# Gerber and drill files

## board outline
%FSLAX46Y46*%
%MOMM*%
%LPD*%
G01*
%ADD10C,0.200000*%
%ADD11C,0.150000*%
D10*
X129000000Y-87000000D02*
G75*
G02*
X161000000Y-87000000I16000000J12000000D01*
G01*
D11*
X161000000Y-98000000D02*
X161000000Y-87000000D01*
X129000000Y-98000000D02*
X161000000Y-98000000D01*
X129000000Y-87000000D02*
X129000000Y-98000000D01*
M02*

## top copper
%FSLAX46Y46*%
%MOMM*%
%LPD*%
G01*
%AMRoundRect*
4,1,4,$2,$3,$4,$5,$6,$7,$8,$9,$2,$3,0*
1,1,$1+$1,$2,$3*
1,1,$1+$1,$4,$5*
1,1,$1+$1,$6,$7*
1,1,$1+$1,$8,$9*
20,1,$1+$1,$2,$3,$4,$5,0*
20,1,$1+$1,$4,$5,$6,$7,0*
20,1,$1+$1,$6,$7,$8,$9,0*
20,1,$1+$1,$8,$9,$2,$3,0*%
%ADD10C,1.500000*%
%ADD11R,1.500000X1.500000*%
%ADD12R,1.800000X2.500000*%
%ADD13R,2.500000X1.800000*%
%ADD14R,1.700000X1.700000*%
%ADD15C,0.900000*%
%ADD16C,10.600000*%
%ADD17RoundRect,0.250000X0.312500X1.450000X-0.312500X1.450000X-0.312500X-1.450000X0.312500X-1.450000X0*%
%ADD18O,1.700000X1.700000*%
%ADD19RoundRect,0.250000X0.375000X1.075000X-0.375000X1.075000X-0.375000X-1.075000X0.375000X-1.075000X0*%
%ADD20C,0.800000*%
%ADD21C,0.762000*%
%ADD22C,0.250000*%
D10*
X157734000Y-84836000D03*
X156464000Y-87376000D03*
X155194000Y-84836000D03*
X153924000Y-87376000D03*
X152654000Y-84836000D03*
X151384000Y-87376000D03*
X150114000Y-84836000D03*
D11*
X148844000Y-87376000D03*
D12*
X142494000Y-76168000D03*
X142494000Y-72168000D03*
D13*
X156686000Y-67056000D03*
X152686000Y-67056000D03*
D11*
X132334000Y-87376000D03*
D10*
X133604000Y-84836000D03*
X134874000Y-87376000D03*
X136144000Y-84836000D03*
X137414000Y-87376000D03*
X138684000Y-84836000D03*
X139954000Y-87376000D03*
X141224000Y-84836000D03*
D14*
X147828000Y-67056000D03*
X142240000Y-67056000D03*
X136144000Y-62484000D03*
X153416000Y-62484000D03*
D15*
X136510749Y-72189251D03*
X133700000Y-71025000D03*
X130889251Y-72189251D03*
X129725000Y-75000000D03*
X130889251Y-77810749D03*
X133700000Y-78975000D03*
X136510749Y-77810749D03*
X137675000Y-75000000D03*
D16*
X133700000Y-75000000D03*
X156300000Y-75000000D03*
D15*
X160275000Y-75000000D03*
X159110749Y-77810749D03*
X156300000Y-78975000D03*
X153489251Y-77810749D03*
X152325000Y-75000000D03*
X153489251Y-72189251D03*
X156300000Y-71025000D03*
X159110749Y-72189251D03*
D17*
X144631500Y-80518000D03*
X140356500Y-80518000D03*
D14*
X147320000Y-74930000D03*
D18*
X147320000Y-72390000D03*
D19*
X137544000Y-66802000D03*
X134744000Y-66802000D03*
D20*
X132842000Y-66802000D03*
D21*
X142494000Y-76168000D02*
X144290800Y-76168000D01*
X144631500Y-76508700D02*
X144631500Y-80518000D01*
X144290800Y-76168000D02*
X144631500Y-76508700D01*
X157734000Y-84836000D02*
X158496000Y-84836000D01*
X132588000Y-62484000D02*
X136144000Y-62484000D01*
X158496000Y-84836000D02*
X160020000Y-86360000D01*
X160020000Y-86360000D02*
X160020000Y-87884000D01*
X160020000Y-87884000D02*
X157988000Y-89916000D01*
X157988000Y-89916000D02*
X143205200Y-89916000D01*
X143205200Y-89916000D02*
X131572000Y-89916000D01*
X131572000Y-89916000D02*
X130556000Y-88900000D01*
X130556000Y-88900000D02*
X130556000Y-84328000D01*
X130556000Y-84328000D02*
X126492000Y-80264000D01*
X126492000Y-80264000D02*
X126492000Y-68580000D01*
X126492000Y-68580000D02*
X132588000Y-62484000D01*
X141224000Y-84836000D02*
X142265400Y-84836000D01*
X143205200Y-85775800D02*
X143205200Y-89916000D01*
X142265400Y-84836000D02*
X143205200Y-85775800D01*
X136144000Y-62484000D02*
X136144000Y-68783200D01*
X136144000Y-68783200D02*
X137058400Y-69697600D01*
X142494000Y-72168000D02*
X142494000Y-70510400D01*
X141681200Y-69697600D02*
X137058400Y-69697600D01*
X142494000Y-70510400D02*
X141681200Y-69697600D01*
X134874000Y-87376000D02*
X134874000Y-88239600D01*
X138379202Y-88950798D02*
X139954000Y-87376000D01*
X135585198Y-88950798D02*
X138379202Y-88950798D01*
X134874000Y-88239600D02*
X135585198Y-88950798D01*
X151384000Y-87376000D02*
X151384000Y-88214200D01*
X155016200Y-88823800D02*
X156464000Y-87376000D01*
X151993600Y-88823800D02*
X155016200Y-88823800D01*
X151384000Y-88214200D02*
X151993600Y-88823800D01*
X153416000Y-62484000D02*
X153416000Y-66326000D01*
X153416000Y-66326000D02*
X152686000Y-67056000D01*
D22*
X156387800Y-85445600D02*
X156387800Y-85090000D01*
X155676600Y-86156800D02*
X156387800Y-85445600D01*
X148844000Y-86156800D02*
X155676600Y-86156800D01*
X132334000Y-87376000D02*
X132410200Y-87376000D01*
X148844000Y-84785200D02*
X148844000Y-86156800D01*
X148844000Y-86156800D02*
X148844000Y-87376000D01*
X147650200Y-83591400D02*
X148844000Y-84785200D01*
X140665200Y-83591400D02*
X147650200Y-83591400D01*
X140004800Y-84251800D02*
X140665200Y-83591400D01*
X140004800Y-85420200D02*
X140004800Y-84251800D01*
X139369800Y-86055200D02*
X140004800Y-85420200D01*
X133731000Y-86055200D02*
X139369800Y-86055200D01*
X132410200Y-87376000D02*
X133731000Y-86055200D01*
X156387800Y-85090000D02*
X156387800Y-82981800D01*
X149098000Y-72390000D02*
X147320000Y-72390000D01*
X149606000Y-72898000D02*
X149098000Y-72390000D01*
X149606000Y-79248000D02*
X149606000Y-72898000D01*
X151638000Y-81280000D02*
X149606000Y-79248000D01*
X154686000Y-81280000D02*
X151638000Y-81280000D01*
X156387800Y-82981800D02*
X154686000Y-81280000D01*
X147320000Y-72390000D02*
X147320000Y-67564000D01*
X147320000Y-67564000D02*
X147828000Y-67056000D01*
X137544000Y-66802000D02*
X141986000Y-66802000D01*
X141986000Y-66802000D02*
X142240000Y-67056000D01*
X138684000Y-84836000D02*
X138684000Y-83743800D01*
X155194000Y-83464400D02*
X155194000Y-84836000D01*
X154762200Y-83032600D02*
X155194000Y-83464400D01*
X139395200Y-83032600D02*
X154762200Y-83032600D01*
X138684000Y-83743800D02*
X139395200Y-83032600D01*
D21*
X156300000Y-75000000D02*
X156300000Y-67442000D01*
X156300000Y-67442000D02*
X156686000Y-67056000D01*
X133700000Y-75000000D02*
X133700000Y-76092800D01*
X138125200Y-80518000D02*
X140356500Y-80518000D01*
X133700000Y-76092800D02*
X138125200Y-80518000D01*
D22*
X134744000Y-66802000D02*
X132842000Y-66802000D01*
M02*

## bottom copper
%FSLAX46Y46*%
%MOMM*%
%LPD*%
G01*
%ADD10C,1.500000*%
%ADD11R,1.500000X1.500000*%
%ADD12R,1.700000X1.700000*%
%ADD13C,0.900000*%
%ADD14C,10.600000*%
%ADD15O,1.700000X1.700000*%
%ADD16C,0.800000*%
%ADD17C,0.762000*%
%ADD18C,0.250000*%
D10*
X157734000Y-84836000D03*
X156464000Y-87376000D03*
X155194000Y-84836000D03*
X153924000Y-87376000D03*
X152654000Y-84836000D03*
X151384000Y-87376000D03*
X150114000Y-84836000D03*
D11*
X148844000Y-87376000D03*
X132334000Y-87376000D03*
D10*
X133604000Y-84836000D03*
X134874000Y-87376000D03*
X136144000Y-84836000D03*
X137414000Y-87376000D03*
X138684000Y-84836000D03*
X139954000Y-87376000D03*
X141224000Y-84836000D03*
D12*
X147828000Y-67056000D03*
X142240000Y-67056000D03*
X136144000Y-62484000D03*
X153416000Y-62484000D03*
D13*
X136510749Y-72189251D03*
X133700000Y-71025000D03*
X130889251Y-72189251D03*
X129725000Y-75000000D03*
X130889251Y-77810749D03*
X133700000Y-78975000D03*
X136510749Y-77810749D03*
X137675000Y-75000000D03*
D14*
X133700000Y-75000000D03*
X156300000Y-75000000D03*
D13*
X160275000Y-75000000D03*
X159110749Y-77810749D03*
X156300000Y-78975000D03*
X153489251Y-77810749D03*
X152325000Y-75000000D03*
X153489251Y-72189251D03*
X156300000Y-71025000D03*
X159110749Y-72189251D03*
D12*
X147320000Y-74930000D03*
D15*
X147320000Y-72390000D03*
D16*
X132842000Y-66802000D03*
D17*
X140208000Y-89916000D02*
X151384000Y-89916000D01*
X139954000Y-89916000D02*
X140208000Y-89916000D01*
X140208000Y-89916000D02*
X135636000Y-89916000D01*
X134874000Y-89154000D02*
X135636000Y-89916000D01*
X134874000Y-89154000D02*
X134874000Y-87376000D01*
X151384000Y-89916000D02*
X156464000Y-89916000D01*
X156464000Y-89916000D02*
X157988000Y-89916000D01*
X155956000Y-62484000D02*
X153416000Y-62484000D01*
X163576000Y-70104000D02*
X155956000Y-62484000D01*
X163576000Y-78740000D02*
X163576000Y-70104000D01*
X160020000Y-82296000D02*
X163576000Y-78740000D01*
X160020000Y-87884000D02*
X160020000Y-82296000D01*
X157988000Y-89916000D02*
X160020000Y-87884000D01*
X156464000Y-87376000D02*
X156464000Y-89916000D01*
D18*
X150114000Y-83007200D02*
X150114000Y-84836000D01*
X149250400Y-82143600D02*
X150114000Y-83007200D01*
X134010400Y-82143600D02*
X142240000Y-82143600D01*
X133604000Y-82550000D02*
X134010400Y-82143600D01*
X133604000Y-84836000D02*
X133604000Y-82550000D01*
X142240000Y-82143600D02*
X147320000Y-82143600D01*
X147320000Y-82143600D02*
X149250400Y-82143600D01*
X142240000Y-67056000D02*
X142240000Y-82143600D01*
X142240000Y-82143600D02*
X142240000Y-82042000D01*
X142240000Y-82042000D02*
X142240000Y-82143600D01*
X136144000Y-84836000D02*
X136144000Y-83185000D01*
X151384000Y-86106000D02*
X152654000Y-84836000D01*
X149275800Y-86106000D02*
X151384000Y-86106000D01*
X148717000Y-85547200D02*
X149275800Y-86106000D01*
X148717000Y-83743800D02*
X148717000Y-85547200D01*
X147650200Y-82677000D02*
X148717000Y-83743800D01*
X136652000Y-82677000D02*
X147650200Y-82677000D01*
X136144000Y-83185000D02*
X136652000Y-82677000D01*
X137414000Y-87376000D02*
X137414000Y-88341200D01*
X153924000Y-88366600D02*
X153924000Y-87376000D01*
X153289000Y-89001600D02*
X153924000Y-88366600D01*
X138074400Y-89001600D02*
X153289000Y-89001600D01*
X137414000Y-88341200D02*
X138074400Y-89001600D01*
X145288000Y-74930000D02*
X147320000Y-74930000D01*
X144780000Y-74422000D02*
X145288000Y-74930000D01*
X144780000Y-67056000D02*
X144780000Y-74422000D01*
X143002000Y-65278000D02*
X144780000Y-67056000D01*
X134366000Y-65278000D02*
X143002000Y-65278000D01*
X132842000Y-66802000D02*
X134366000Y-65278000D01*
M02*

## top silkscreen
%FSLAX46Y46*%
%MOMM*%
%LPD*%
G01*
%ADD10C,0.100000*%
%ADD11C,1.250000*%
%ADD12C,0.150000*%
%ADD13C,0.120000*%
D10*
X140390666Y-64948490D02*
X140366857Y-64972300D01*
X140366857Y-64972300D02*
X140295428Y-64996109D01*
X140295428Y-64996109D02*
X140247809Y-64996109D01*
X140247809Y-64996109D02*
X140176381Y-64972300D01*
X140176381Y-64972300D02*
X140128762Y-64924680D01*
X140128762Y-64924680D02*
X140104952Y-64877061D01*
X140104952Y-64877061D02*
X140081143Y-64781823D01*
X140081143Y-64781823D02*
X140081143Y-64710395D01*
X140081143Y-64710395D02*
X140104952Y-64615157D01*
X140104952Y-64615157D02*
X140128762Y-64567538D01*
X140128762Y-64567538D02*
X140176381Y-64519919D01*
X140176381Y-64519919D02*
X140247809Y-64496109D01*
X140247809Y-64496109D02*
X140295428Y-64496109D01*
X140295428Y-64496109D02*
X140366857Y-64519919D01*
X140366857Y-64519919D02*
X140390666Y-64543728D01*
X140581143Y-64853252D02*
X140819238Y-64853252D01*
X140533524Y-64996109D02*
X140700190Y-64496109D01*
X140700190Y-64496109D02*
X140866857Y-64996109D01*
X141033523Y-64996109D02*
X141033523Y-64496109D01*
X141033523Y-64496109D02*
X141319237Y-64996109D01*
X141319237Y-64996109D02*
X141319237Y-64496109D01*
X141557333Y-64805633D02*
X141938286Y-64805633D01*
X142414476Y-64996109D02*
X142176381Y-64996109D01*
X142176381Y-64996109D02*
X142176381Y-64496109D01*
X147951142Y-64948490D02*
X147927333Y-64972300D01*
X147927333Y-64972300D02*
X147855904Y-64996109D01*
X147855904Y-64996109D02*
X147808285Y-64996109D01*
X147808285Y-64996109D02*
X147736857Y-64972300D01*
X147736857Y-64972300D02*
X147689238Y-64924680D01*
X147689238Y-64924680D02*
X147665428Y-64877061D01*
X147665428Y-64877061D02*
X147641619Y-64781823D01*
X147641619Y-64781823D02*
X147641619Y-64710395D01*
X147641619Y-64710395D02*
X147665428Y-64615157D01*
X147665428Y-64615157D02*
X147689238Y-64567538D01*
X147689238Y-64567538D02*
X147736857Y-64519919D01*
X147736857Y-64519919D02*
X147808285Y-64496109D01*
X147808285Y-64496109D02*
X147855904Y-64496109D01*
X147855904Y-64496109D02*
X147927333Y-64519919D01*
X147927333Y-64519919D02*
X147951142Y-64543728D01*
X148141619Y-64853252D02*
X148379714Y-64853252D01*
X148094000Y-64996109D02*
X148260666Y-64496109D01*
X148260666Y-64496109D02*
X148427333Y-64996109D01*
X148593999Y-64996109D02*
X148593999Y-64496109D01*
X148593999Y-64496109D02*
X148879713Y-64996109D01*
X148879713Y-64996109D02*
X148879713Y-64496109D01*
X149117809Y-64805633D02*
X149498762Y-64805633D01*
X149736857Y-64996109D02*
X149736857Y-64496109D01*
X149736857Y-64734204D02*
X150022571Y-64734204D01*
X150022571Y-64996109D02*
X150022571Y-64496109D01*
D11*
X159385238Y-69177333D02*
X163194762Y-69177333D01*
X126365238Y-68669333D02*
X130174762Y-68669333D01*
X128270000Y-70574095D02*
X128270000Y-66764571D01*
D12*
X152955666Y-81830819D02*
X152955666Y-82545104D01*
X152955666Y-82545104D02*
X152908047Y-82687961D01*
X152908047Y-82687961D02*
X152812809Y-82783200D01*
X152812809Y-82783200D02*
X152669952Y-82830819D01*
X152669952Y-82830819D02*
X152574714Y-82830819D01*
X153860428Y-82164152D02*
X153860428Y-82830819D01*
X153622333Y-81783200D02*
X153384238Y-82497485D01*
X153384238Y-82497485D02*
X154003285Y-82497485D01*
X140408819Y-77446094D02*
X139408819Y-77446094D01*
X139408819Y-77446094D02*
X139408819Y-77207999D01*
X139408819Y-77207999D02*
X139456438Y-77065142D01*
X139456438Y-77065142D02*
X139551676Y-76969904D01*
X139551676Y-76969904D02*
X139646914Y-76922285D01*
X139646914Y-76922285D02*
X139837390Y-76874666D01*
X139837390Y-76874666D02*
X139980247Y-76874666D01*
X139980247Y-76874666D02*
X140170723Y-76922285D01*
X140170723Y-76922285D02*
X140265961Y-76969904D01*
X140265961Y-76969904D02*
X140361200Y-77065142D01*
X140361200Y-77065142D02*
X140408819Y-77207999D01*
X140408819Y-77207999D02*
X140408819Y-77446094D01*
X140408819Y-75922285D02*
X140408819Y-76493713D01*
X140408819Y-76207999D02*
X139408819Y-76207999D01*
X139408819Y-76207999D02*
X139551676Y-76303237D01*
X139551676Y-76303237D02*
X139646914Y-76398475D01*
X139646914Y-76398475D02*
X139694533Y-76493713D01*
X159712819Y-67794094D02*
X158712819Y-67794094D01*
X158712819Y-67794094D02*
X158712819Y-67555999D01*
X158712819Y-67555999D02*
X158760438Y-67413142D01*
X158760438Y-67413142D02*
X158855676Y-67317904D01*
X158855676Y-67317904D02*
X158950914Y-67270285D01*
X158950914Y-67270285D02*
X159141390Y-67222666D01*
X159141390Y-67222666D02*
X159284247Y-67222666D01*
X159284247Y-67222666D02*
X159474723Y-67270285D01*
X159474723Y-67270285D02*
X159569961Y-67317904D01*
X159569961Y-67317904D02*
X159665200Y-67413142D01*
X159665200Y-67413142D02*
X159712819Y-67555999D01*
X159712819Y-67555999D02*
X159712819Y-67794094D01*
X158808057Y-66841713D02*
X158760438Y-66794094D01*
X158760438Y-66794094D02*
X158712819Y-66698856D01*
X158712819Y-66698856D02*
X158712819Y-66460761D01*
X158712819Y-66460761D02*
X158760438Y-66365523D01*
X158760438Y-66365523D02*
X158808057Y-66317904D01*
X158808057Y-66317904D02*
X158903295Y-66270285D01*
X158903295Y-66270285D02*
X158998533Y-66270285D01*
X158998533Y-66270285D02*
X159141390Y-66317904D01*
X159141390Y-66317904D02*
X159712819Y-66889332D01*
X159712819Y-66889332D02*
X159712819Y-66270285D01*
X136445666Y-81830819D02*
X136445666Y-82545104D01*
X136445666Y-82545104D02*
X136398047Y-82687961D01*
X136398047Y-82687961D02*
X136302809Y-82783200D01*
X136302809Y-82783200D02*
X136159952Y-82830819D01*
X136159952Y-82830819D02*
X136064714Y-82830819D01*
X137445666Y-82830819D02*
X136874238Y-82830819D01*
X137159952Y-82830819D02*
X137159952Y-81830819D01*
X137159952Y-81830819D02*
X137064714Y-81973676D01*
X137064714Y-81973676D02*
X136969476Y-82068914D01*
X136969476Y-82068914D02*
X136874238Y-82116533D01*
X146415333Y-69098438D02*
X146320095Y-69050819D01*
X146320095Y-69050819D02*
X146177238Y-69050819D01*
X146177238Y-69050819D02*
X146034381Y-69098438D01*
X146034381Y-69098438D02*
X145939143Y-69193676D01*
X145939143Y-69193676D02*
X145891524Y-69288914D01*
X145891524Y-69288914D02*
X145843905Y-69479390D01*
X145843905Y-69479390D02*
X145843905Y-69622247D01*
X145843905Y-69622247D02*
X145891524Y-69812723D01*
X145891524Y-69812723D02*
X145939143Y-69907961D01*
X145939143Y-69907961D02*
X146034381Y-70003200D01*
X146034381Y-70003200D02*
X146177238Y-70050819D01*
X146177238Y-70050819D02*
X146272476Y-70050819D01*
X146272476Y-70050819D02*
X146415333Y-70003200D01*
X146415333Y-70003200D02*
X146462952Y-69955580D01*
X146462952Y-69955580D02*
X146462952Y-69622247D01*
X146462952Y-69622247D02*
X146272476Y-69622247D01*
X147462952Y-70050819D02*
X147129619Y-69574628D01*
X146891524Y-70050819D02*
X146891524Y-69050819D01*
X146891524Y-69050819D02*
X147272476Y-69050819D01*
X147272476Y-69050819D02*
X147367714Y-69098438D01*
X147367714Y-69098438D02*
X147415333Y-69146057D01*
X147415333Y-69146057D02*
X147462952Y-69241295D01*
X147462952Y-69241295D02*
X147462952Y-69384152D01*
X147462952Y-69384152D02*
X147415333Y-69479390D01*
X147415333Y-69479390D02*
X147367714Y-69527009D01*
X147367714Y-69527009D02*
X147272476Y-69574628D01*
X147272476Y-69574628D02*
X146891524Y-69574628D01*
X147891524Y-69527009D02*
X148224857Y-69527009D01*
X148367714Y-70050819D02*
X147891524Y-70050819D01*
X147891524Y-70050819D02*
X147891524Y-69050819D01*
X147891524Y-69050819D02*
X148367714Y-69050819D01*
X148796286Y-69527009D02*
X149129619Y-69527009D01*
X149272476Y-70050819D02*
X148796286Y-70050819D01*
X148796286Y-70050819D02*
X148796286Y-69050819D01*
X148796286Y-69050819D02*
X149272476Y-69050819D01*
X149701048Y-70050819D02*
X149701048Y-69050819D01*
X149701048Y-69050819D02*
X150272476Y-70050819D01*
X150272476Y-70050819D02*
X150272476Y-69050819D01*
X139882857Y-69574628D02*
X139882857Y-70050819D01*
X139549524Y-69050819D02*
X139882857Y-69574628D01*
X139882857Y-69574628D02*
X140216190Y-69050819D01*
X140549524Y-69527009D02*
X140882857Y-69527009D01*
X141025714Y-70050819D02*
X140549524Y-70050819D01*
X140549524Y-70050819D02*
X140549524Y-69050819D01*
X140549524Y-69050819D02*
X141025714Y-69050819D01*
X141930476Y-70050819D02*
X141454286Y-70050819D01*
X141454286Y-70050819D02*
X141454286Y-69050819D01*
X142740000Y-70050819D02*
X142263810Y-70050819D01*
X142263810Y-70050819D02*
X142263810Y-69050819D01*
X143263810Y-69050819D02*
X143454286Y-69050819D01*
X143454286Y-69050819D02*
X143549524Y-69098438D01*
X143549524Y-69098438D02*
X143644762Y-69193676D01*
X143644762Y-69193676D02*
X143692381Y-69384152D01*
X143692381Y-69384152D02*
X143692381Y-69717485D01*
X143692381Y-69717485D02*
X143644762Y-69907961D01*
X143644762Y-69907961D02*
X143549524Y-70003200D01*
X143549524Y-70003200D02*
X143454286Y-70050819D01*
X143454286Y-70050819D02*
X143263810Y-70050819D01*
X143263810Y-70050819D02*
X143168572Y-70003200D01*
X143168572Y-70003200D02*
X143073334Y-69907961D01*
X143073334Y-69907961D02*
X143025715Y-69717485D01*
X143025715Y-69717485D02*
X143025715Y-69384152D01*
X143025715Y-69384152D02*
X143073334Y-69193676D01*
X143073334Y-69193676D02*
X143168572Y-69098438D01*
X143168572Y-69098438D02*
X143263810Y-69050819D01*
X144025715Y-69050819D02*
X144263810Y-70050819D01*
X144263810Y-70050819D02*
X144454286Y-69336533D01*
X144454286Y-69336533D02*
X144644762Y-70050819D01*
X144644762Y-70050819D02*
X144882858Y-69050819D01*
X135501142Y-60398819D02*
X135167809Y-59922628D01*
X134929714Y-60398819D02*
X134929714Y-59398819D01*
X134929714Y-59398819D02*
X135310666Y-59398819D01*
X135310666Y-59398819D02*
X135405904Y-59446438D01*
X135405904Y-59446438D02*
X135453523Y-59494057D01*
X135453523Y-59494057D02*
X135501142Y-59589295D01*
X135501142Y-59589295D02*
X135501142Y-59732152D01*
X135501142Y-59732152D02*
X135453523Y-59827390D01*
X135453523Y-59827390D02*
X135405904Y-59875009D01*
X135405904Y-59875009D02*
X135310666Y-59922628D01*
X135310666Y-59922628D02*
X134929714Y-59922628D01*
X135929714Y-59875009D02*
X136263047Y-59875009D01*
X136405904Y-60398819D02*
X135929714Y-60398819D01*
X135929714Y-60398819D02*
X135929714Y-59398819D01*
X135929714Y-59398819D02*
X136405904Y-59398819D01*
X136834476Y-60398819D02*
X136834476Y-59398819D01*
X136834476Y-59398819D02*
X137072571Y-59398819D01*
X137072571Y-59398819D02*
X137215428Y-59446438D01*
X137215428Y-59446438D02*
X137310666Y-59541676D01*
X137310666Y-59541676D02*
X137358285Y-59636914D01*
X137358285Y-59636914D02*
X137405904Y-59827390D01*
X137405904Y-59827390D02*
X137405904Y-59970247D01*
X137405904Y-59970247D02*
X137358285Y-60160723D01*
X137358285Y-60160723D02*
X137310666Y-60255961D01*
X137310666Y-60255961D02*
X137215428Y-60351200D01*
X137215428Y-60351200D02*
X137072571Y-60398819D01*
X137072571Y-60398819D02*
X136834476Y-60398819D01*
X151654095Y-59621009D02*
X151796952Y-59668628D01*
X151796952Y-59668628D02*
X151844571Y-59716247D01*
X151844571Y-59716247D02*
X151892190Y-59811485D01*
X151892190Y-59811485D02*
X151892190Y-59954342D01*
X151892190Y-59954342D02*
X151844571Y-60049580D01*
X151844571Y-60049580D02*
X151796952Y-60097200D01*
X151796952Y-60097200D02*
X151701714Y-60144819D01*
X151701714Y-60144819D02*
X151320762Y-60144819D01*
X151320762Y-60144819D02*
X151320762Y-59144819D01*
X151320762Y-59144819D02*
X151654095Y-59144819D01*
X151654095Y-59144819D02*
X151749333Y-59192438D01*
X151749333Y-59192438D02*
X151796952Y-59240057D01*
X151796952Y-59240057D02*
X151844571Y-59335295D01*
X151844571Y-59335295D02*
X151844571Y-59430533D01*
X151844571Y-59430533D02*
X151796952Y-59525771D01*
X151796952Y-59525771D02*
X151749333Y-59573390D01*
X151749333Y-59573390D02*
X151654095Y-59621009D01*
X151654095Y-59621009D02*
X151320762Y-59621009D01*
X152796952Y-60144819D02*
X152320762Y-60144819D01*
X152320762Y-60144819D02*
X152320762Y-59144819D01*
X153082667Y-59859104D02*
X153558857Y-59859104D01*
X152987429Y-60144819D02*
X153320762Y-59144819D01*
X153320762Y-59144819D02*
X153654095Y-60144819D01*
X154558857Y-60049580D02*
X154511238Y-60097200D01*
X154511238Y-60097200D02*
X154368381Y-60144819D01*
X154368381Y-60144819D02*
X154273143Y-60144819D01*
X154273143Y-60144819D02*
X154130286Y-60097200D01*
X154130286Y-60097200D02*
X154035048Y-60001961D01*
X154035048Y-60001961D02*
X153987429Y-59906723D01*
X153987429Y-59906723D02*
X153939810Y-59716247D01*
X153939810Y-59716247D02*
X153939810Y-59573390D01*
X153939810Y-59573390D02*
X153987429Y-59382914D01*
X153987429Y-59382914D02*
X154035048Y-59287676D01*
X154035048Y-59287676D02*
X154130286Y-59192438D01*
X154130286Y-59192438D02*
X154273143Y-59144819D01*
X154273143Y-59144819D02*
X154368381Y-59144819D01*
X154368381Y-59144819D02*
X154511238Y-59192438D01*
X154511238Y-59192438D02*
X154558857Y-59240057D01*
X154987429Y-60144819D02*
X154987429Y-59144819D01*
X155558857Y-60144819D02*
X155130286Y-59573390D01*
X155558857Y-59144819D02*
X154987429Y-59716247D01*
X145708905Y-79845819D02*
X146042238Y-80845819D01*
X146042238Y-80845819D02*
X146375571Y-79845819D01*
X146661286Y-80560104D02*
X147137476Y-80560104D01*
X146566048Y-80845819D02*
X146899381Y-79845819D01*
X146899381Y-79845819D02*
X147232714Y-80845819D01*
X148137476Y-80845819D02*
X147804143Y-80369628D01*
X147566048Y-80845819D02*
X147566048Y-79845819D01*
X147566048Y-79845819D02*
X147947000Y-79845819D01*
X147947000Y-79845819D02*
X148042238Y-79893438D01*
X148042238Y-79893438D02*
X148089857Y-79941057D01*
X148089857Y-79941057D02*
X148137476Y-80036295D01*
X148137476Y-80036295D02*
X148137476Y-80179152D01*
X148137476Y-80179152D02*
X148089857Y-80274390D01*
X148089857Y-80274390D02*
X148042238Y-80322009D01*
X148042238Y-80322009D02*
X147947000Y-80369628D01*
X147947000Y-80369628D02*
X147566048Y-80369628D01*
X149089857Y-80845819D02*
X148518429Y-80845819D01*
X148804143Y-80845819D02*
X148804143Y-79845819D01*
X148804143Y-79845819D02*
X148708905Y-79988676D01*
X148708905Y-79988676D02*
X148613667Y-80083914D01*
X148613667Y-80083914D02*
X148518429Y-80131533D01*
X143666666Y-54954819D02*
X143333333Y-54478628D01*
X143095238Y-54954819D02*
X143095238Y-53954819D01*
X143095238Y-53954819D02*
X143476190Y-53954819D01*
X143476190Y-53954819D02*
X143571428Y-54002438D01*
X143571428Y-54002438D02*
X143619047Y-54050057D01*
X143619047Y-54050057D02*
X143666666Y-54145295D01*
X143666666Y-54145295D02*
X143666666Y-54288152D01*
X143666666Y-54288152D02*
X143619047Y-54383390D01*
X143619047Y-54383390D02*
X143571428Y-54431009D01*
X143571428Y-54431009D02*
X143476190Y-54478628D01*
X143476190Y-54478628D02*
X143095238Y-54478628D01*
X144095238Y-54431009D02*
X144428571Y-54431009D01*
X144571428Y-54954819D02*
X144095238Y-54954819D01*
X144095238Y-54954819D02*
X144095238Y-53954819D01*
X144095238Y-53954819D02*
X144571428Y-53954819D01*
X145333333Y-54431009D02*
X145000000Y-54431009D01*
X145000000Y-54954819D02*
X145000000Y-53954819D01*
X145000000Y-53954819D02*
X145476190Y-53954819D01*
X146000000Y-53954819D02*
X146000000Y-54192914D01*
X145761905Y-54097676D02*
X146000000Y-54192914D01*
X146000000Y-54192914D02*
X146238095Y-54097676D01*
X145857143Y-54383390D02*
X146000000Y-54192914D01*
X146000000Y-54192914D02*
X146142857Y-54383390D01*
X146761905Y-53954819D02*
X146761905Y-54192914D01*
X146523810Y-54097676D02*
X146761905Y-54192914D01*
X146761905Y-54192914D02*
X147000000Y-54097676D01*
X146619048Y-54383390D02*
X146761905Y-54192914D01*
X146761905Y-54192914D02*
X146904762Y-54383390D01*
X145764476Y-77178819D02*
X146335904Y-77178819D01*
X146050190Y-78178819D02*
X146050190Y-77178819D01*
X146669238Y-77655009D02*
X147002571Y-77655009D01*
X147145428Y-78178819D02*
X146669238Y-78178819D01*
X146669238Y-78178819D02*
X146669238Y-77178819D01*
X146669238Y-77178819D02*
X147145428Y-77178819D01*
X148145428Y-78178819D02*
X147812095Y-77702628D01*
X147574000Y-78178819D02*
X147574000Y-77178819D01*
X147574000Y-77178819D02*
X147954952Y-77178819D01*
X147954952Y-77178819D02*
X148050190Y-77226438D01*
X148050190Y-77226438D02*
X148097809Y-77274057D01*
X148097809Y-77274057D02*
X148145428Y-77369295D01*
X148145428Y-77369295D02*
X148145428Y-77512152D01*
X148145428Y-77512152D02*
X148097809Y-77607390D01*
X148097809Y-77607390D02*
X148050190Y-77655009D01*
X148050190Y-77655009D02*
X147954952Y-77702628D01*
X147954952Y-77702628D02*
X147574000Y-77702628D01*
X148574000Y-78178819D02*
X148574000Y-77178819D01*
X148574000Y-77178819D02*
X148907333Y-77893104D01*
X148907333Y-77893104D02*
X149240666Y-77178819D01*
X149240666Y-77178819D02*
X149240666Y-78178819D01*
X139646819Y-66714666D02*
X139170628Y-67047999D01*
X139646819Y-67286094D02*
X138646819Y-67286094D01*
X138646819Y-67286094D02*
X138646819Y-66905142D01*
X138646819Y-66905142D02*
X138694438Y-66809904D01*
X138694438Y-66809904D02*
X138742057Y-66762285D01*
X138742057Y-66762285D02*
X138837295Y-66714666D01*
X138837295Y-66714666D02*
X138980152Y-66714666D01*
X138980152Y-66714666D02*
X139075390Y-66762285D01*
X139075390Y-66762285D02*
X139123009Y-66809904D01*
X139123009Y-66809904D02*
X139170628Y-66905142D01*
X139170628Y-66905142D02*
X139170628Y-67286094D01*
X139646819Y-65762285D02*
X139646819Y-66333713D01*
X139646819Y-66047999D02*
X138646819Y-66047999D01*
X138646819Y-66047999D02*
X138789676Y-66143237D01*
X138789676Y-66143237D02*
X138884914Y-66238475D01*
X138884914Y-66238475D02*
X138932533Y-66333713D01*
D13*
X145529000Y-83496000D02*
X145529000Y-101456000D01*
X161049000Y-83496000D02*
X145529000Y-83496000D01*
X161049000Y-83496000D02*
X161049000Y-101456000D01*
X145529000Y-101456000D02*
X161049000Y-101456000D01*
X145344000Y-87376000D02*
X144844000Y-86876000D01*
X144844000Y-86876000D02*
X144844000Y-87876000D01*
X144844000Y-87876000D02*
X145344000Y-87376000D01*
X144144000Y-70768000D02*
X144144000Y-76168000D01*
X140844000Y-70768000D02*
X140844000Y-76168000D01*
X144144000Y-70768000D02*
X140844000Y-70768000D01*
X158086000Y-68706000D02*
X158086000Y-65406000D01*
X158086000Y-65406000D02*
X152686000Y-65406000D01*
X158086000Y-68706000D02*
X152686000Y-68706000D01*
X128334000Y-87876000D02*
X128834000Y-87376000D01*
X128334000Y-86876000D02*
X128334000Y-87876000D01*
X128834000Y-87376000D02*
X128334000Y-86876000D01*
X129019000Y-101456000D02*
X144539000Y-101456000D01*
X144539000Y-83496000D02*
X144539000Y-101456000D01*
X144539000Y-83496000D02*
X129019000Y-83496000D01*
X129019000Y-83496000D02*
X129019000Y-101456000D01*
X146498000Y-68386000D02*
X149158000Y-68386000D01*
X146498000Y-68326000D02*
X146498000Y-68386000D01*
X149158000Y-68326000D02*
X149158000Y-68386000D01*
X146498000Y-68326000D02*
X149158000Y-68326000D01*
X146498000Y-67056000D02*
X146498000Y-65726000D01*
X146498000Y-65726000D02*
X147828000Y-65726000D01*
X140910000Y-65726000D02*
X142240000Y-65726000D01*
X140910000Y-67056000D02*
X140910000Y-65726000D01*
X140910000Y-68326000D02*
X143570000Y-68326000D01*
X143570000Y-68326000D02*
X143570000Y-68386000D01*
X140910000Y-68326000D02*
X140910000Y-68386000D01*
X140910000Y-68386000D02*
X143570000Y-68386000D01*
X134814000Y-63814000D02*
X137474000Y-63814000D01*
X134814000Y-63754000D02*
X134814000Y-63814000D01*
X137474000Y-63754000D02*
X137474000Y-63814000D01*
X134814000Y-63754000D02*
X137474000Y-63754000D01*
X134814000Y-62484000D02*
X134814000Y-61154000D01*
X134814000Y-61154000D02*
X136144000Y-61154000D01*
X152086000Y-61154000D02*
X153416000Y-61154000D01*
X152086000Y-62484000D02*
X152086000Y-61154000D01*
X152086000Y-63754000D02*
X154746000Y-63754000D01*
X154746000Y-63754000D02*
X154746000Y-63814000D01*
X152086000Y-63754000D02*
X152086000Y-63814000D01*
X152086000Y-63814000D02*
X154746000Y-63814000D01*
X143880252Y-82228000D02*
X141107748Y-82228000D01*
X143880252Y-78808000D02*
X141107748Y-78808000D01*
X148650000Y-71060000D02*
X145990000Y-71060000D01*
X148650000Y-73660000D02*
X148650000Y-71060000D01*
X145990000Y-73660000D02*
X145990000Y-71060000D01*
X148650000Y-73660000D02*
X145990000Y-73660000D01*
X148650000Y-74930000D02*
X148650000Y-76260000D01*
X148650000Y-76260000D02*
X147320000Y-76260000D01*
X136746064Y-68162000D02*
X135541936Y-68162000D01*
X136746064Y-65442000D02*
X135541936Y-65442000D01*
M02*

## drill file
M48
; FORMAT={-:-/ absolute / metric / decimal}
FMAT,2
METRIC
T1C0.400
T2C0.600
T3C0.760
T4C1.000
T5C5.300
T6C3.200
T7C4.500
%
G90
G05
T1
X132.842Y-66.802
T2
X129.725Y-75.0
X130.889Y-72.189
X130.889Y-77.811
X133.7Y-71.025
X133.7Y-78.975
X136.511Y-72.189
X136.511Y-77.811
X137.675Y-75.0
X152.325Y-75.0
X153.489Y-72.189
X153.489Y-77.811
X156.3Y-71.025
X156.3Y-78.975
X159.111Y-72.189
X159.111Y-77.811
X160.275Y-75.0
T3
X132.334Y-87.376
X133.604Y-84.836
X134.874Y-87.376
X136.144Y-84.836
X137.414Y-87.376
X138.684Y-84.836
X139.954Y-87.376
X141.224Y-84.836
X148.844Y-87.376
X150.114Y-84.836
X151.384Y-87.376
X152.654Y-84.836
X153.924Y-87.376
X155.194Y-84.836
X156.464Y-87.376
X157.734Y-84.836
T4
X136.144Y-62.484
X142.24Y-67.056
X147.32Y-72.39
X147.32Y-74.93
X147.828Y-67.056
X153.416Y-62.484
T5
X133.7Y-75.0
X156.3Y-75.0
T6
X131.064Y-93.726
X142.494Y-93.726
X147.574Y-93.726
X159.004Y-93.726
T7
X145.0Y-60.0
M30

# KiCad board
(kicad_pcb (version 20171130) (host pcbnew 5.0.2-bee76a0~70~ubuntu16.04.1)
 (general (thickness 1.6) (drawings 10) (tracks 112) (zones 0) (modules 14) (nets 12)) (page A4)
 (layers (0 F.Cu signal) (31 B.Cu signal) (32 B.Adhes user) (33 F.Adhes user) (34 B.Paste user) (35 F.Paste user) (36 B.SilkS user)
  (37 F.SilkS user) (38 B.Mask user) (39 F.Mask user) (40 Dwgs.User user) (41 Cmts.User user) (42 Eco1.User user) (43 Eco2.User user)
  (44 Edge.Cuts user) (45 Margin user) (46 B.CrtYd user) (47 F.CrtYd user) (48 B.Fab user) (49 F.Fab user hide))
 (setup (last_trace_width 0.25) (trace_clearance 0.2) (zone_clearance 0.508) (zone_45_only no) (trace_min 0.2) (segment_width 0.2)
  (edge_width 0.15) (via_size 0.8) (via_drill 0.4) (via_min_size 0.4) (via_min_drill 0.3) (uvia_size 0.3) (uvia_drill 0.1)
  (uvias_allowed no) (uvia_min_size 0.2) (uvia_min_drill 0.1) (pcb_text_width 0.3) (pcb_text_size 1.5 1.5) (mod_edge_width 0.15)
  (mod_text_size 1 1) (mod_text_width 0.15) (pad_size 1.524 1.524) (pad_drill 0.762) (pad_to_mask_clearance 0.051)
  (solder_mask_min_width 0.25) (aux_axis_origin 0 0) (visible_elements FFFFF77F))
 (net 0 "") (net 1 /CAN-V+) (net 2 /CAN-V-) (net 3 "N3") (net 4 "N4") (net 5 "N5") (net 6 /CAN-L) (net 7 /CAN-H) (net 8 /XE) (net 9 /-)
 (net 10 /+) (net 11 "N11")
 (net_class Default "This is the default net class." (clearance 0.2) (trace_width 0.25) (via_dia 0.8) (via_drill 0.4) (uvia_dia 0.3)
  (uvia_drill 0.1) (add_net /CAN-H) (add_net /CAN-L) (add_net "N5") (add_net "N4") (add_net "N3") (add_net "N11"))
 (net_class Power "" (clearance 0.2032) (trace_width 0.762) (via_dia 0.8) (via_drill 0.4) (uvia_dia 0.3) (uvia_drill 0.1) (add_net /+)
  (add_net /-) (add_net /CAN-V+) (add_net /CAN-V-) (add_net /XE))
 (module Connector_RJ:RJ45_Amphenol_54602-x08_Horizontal (layer F.Cu) (at 148.844 87.376)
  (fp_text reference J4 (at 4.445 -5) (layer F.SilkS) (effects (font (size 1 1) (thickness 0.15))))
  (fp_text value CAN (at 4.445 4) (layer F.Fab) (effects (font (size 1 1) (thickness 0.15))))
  (fp_line (start -3.315 -3.88) (end -3.315 14.08) (layer F.SilkS) (width 0.12))
  (fp_line (start 12.205 -3.88) (end -3.315 -3.88) (layer F.SilkS) (width 0.12))
  (fp_line (start 12.205 -3.88) (end 12.205 14.08) (layer F.SilkS) (width 0.12))
  (fp_line (start -3.315 14.08) (end 12.205 14.08) (layer F.SilkS) (width 0.12))
  (fp_line (start -3.5 0) (end -4 -0.5) (layer F.SilkS) (width 0.12))
  (fp_line (start -4 -0.5) (end -4 0.5) (layer F.SilkS) (width 0.12))
  (fp_line (start -4 0.5) (end -3.5 0) (layer F.SilkS) (width 0.12))
  (pad 8 thru_hole circle (at 8.89 -2.54) (size 1.5 1.5) (drill 0.76) (layers *.Cu *.Mask) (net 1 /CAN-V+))
  (pad 7 thru_hole circle (at 7.62 0) (size 1.5 1.5) (drill 0.76) (layers *.Cu *.Mask) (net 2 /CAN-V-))
  (pad 6 thru_hole circle (at 6.35 -2.54) (size 1.5 1.5) (drill 0.76) (layers *.Cu *.Mask) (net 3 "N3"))
  (pad 5 thru_hole circle (at 5.08 0) (size 1.5 1.5) (drill 0.76) (layers *.Cu *.Mask) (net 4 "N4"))
  (pad 4 thru_hole circle (at 3.81 -2.54) (size 1.5 1.5) (drill 0.76) (layers *.Cu *.Mask) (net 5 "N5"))
  (pad 3 thru_hole circle (at 2.54 0) (size 1.5 1.5) (drill 0.76) (layers *.Cu *.Mask) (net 2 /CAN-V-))
  (pad 2 thru_hole circle (at 1.27 -2.54) (size 1.5 1.5) (drill 0.76) (layers *.Cu *.Mask) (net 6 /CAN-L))
  (pad 1 thru_hole rect (at 0 0) (size 1.5 1.5) (drill 0.76) (layers *.Cu *.Mask) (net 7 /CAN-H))
  (pad "" np_thru_hole circle (at -1.27 6.35) (size 3.2 3.2) (drill 3.2) (layers *.Cu *.Mask))
  (pad "" np_thru_hole circle (at 10.16 6.35) (size 3.2 3.2) (drill 3.2) (layers *.Cu *.Mask)))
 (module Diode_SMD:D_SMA (layer F.Cu) (at 142.494 74.168 270)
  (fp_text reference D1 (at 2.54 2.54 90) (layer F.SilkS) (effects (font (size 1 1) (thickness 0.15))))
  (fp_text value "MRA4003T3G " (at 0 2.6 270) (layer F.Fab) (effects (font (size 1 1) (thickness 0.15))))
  (fp_line (start -3.4 -1.65) (end 2 -1.65) (layer F.SilkS) (width 0.12))
  (fp_line (start -3.4 1.65) (end 2 1.65) (layer F.SilkS) (width 0.12))
  (fp_line (start -3.4 -1.65) (end -3.4 1.65) (layer F.SilkS) (width 0.12))
  (pad 2 smd rect (at 2 0 270) (size 2.5 1.8) (layers F.Cu F.Paste F.Mask) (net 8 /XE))
  (pad 1 smd rect (at -2 0 270) (size 2.5 1.8) (layers F.Cu F.Paste F.Mask) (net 1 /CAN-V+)))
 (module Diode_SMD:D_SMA (layer F.Cu) (at 154.686 67.056 180)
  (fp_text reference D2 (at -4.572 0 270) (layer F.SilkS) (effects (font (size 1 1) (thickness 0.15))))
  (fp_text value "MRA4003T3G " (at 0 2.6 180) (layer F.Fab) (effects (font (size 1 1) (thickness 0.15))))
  (fp_line (start -3.4 -1.65) (end -3.4 1.65) (layer F.SilkS) (width 0.12))
  (fp_line (start -3.4 1.65) (end 2 1.65) (layer F.SilkS) (width 0.12))
  (fp_line (start -3.4 -1.65) (end 2 -1.65) (layer F.SilkS) (width 0.12))
  (pad 1 smd rect (at -2 0 180) (size 2.5 1.8) (layers F.Cu F.Paste F.Mask) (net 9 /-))
  (pad 2 smd rect (at 2 0 180) (size 2.5 1.8) (layers F.Cu F.Paste F.Mask) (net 2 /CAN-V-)))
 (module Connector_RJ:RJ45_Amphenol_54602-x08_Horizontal (layer F.Cu) (at 132.334 87.376)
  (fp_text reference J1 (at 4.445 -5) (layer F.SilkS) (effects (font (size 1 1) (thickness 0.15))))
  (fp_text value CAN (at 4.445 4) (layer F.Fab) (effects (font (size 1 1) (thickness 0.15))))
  (fp_line (start -4 0.5) (end -3.5 0) (layer F.SilkS) (width 0.12))
  (fp_line (start -4 -0.5) (end -4 0.5) (layer F.SilkS) (width 0.12))
  (fp_line (start -3.5 0) (end -4 -0.5) (layer F.SilkS) (width 0.12))
  (fp_line (start -3.315 14.08) (end 12.205 14.08) (layer F.SilkS) (width 0.12))
  (fp_line (start 12.205 -3.88) (end 12.205 14.08) (layer F.SilkS) (width 0.12))
  (fp_line (start 12.205 -3.88) (end -3.315 -3.88) (layer F.SilkS) (width 0.12))
  (fp_line (start -3.315 -3.88) (end -3.315 14.08) (layer F.SilkS) (width 0.12))
  (pad "" np_thru_hole circle (at 10.16 6.35) (size 3.2 3.2) (drill 3.2) (layers *.Cu *.Mask))
  (pad "" np_thru_hole circle (at -1.27 6.35) (size 3.2 3.2) (drill 3.2) (layers *.Cu *.Mask))
  (pad 1 thru_hole rect (at 0 0) (size 1.5 1.5) (drill 0.76) (layers *.Cu *.Mask) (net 7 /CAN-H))
  (pad 2 thru_hole circle (at 1.27 -2.54) (size 1.5 1.5) (drill 0.76) (layers *.Cu *.Mask) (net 6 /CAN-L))
  (pad 3 thru_hole circle (at 2.54 0) (size 1.5 1.5) (drill 0.76) (layers *.Cu *.Mask) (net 2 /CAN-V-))
  (pad 4 thru_hole circle (at 3.81 -2.54) (size 1.5 1.5) (drill 0.76) (layers *.Cu *.Mask) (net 5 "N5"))
  (pad 5 thru_hole circle (at 5.08 0) (size 1.5 1.5) (drill 0.76) (layers *.Cu *.Mask) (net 4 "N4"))
  (pad 6 thru_hole circle (at 6.35 -2.54) (size 1.5 1.5) (drill 0.76) (layers *.Cu *.Mask) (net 3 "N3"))
  (pad 7 thru_hole circle (at 7.62 0) (size 1.5 1.5) (drill 0.76) (layers *.Cu *.Mask) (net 2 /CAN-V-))
  (pad 8 thru_hole circle (at 8.89 -2.54) (size 1.5 1.5) (drill 0.76) (layers *.Cu *.Mask) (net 1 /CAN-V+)))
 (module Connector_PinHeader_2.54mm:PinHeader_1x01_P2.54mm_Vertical (layer F.Cu) (at 147.828 67.056)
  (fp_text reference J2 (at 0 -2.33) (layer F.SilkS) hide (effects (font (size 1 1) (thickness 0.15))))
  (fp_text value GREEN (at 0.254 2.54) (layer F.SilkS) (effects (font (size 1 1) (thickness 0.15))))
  (fp_line (start -1.33 1.33) (end 1.33 1.33) (layer F.SilkS) (width 0.12))
  (fp_line (start -1.33 1.27) (end -1.33 1.33) (layer F.SilkS) (width 0.12))
  (fp_line (start 1.33 1.27) (end 1.33 1.33) (layer F.SilkS) (width 0.12))
  (fp_line (start -1.33 1.27) (end 1.33 1.27) (layer F.SilkS) (width 0.12))
  (fp_line (start -1.33 0) (end -1.33 -1.33) (layer F.SilkS) (width 0.12))
  (fp_line (start -1.33 -1.33) (end 0 -1.33) (layer F.SilkS) (width 0.12))
  (pad 1 thru_hole rect (at 0 0) (size 1.7 1.7) (drill 1) (layers *.Cu *.Mask) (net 7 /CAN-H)))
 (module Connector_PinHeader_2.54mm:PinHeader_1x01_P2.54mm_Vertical (layer F.Cu) (at 142.24 67.056)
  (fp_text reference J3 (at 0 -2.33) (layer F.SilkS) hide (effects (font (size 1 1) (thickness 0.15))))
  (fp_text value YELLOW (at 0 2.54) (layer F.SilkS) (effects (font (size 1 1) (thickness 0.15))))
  (fp_line (start -1.33 -1.33) (end 0 -1.33) (layer F.SilkS) (width 0.12))
  (fp_line (start -1.33 0) (end -1.33 -1.33) (layer F.SilkS) (width 0.12))
  (fp_line (start -1.33 1.27) (end 1.33 1.27) (layer F.SilkS) (width 0.12))
  (fp_line (start 1.33 1.27) (end 1.33 1.33) (layer F.SilkS) (width 0.12))
  (fp_line (start -1.33 1.27) (end -1.33 1.33) (layer F.SilkS) (width 0.12))
  (fp_line (start -1.33 1.33) (end 1.33 1.33) (layer F.SilkS) (width 0.12))
  (pad 1 thru_hole rect (at 0 0) (size 1.7 1.7) (drill 1) (layers *.Cu *.Mask) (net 6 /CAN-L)))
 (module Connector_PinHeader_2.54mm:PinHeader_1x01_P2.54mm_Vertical (layer F.Cu) (at 136.144 62.484)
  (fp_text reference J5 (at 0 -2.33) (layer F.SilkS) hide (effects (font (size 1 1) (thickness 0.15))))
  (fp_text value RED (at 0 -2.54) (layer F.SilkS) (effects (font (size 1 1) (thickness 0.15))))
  (fp_line (start -1.33 1.33) (end 1.33 1.33) (layer F.SilkS) (width 0.12))
  (fp_line (start -1.33 1.27) (end -1.33 1.33) (layer F.SilkS) (width 0.12))
  (fp_line (start 1.33 1.27) (end 1.33 1.33) (layer F.SilkS) (width 0.12))
  (fp_line (start -1.33 1.27) (end 1.33 1.27) (layer F.SilkS) (width 0.12))
  (fp_line (start -1.33 0) (end -1.33 -1.33) (layer F.SilkS) (width 0.12))
  (fp_line (start -1.33 -1.33) (end 0 -1.33) (layer F.SilkS) (width 0.12))
  (pad 1 thru_hole rect (at 0 0) (size 1.7 1.7) (drill 1) (layers *.Cu *.Mask) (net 1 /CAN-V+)))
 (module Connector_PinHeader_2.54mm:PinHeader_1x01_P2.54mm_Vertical (layer F.Cu) (at 153.416 62.484)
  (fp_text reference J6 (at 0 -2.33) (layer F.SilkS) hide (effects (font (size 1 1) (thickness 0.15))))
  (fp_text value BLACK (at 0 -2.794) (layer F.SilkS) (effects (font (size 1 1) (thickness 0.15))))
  (fp_line (start -1.33 -1.33) (end 0 -1.33) (layer F.SilkS) (width 0.12))
  (fp_line (start -1.33 0) (end -1.33 -1.33) (layer F.SilkS) (width 0.12))
  (fp_line (start -1.33 1.27) (end 1.33 1.27) (layer F.SilkS) (width 0.12))
  (fp_line (start 1.33 1.27) (end 1.33 1.33) (layer F.SilkS) (width 0.12))
  (fp_line (start -1.33 1.27) (end -1.33 1.33) (layer F.SilkS) (width 0.12))
  (fp_line (start -1.33 1.33) (end 1.33 1.33) (layer F.SilkS) (width 0.12))
  (pad 1 thru_hole rect (at 0 0) (size 1.7 1.7) (drill 1) (layers *.Cu *.Mask) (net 2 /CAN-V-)))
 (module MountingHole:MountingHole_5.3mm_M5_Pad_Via (layer F.Cu) (at 133.7 75)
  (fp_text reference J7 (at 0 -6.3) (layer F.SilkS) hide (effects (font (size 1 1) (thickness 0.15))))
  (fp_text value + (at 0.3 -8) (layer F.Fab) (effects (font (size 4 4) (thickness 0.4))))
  (pad 1 thru_hole circle (at 2.810749 -2.810749) (size 0.9 0.9) (drill 0.6) (layers *.Cu *.Mask) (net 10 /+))
  (pad 1 thru_hole circle (at 0 -3.975) (size 0.9 0.9) (drill 0.6) (layers *.Cu *.Mask) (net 10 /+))
  (pad 1 thru_hole circle (at -2.810749 -2.810749) (size 0.9 0.9) (drill 0.6) (layers *.Cu *.Mask) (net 10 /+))
  (pad 1 thru_hole circle (at -3.975 0) (size 0.9 0.9) (drill 0.6) (layers *.Cu *.Mask) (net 10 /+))
  (pad 1 thru_hole circle (at -2.810749 2.810749) (size 0.9 0.9) (drill 0.6) (layers *.Cu *.Mask) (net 10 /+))
  (pad 1 thru_hole circle (at 0 3.975) (size 0.9 0.9) (drill 0.6) (layers *.Cu *.Mask) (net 10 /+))
  (pad 1 thru_hole circle (at 2.810749 2.810749) (size 0.9 0.9) (drill 0.6) (layers *.Cu *.Mask) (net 10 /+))
  (pad 1 thru_hole circle (at 3.975 0) (size 0.9 0.9) (drill 0.6) (layers *.Cu *.Mask) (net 10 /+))
  (pad 1 thru_hole circle (at 0 0) (size 10.6 10.6) (drill 5.3) (layers *.Cu *.Mask) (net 10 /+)))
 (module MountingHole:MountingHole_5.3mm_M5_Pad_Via (layer F.Cu) (at 156.3 75)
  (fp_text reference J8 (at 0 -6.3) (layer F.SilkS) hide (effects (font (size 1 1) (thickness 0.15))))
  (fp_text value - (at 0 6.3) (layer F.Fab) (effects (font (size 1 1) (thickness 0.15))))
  (pad 1 thru_hole circle (at 0 0) (size 10.6 10.6) (drill 5.3) (layers *.Cu *.Mask) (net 9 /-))
  (pad 1 thru_hole circle (at 3.975 0) (size 0.9 0.9) (drill 0.6) (layers *.Cu *.Mask) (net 9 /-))
  (pad 1 thru_hole circle (at 2.810749 2.810749) (size 0.9 0.9) (drill 0.6) (layers *.Cu *.Mask) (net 9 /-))
  (pad 1 thru_hole circle (at 0 3.975) (size 0.9 0.9) (drill 0.6) (layers *.Cu *.Mask) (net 9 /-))
  (pad 1 thru_hole circle (at -2.810749 2.810749) (size 0.9 0.9) (drill 0.6) (layers *.Cu *.Mask) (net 9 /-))
  (pad 1 thru_hole circle (at -3.975 0) (size 0.9 0.9) (drill 0.6) (layers *.Cu *.Mask) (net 9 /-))
  (pad 1 thru_hole circle (at -2.810749 -2.810749) (size 0.9 0.9) (drill 0.6) (layers *.Cu *.Mask) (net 9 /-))
  (pad 1 thru_hole circle (at 0 -3.975) (size 0.9 0.9) (drill 0.6) (layers *.Cu *.Mask) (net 9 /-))
  (pad 1 thru_hole circle (at 2.810749 -2.810749) (size 0.9 0.9) (drill 0.6) (layers *.Cu *.Mask) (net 9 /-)))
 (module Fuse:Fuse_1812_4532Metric (layer F.Cu) (at 142.494 80.518 180)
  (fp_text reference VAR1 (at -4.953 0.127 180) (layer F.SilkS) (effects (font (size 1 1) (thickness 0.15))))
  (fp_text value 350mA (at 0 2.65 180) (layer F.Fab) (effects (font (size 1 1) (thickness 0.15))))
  (fp_line (start -1.386252 -1.71) (end 1.386252 -1.71) (layer F.SilkS) (width 0.12))
  (fp_line (start -1.386252 1.71) (end 1.386252 1.71) (layer F.SilkS) (width 0.12))
  (pad 1 smd roundrect (at -2.1375 0 180) (size 1.125 3.4) (layers F.Cu F.Paste F.Mask) (roundrect_rratio 0.222222) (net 8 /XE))
  (pad 2 smd roundrect (at 2.1375 0 180) (size 1.125 3.4) (layers F.Cu F.Paste F.Mask) (roundrect_rratio 0.222222) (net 10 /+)))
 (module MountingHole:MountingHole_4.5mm (layer F.Cu) (at 145 60)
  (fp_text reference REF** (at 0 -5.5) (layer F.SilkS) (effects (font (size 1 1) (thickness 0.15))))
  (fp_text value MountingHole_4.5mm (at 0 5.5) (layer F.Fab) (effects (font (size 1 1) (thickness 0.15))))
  (pad 1 np_thru_hole circle (at 0 0) (size 4.5 4.5) (drill 4.5) (layers *.Cu *.Mask)))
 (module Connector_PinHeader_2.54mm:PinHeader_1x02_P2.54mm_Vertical (layer F.Cu) (at 147.32 74.93 180)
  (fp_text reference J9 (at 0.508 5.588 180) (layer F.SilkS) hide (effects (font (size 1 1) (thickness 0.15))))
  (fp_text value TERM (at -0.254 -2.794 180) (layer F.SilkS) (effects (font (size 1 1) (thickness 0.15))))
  (fp_line (start -1.33 3.87) (end 1.33 3.87) (layer F.SilkS) (width 0.12))
  (fp_line (start -1.33 1.27) (end -1.33 3.87) (layer F.SilkS) (width 0.12))
  (fp_line (start 1.33 1.27) (end 1.33 3.87) (layer F.SilkS) (width 0.12))
  (fp_line (start -1.33 1.27) (end 1.33 1.27) (layer F.SilkS) (width 0.12))
  (fp_line (start -1.33 0) (end -1.33 -1.33) (layer F.SilkS) (width 0.12))
  (fp_line (start -1.33 -1.33) (end 0 -1.33) (layer F.SilkS) (width 0.12))
  (pad 1 thru_hole rect (at 0 0 180) (size 1.7 1.7) (drill 1) (layers *.Cu *.Mask) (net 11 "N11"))
  (pad 2 thru_hole oval (at 0 2.54 180) (size 1.7 1.7) (drill 1) (layers *.Cu *.Mask) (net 7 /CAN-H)))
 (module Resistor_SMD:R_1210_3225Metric (layer F.Cu) (at 136.144 66.802 180)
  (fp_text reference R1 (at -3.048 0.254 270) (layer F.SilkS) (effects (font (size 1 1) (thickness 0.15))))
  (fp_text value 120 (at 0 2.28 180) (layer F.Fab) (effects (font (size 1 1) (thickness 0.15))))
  (fp_line (start -0.602064 -1.36) (end 0.602064 -1.36) (layer F.SilkS) (width 0.12))
  (fp_line (start -0.602064 1.36) (end 0.602064 1.36) (layer F.SilkS) (width 0.12))
  (pad 1 smd roundrect (at -1.4 0 180) (size 1.25 2.65) (layers F.Cu F.Paste F.Mask) (roundrect_rratio 0.2) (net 6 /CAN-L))
  (pad 2 smd roundrect (at 1.4 0 180) (size 1.25 2.65) (layers F.Cu F.Paste F.Mask) (roundrect_rratio 0.2) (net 11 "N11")))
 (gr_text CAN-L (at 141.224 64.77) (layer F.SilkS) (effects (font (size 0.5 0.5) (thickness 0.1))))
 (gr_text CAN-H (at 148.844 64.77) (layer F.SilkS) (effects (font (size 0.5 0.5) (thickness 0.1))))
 (gr_arc (start 145 75) (end 161 87) (angle -253.7397953) (layer Edge.Cuts) (width 0.2))
 (gr_line (start 161 98) (end 161 87) (angle 90) (layer Edge.Cuts) (width 0.15))
 (gr_line (start 129 98) (end 161 98) (angle 90) (layer Edge.Cuts) (width 0.15))
 (gr_line (start 129 87) (end 129 98) (angle 90) (layer Edge.Cuts) (width 0.15))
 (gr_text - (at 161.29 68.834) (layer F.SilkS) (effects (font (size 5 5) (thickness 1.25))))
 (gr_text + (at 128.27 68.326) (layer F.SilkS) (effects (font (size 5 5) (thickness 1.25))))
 (segment (start 142.494 76.168) (end 144.2908 76.168) (width 0.762) (layer F.Cu) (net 8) (status 400000))
 (segment (start 144.6315 76.5087) (end 144.6315 80.518) (width 0.762) (layer F.Cu) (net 8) (status 800000))
 (segment (start 144.2908 76.168) (end 144.6315 76.5087) (width 0.762) (layer F.Cu) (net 8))
 (segment (start 157.734 84.836) (end 158.496 84.836) (width 0.762) (layer F.Cu) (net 1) (status 400000))
 (segment (start 132.588 62.484) (end 136.144 62.484) (width 0.762) (layer F.Cu) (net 1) (status 800000))
 (segment (start 158.496 84.836) (end 160.02 86.36) (width 0.762) (layer F.Cu) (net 1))
 (segment (start 160.02 86.36) (end 160.02 87.884) (width 0.762) (layer F.Cu) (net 1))
 (segment (start 160.02 87.884) (end 157.988 89.916) (width 0.762) (layer F.Cu) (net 1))
 (segment (start 157.988 89.916) (end 143.2052 89.916) (width 0.762) (layer F.Cu) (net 1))
 (segment (start 143.2052 89.916) (end 131.572 89.916) (width 0.762) (layer F.Cu) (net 1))
 (segment (start 131.572 89.916) (end 130.556 88.9) (width 0.762) (layer F.Cu) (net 1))
 (segment (start 130.556 88.9) (end 130.556 84.328) (width 0.762) (layer F.Cu) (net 1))
 (segment (start 130.556 84.328) (end 126.492 80.264) (width 0.762) (layer F.Cu) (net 1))
 (segment (start 126.492 80.264) (end 126.492 68.58) (width 0.762) (layer F.Cu) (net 1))
 (segment (start 126.492 68.58) (end 132.588 62.484) (width 0.762) (layer F.Cu) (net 1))
 (segment (start 141.224 84.836) (end 142.2654 84.836) (width 0.762) (layer F.Cu) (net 1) (status 400000))
 (segment (start 143.2052 85.7758) (end 143.2052 89.916) (width 0.762) (layer F.Cu) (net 1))
 (segment (start 142.2654 84.836) (end 143.2052 85.7758) (width 0.762) (layer F.Cu) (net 1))
 (segment (start 136.144 62.484) (end 136.144 68.7832) (width 0.762) (layer F.Cu) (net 1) (status 400000))
 (segment (start 136.144 68.7832) (end 137.0584 69.6976) (width 0.762) (layer F.Cu) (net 1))
 (segment (start 142.494 72.168) (end 142.494 70.5104) (width 0.762) (layer F.Cu) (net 1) (status 400000))
 (segment (start 141.6812 69.6976) (end 137.0584 69.6976) (width 0.762) (layer F.Cu) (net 1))
 (segment (start 142.494 70.5104) (end 141.6812 69.6976) (width 0.762) (layer F.Cu) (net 1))
 (segment (start 140.208 89.916) (end 151.384 89.916) (width 0.762) (layer B.Cu) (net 2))
 (segment (start 139.954 89.916) (end 140.208 89.916) (width 0.762) (layer B.Cu) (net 2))
 (segment (start 140.208 89.916) (end 135.636 89.916) (width 0.762) (layer B.Cu) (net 2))
 (segment (start 134.874 89.154) (end 135.636 89.916) (width 0.762) (layer B.Cu) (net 2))
 (segment (start 134.874 89.154) (end 134.874 87.376) (width 0.762) (layer B.Cu) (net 2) (status 800000))
 (segment (start 151.384 89.916) (end 156.464 89.916) (width 0.762) (layer B.Cu) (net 2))
 (segment (start 156.464 89.916) (end 157.988 89.916) (width 0.762) (layer B.Cu) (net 2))
 (segment (start 155.956 62.484) (end 153.416 62.484) (width 0.762) (layer B.Cu) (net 2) (status 800000))
 (segment (start 163.576 70.104) (end 155.956 62.484) (width 0.762) (layer B.Cu) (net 2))
 (segment (start 163.576 78.74) (end 163.576 70.104) (width 0.762) (layer B.Cu) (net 2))
 (segment (start 160.02 82.296) (end 163.576 78.74) (width 0.762) (layer B.Cu) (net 2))
 (segment (start 160.02 87.884) (end 160.02 82.296) (width 0.762) (layer B.Cu) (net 2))
 (segment (start 157.988 89.916) (end 160.02 87.884) (width 0.762) (layer B.Cu) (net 2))
 (segment (start 156.464 87.376) (end 156.464 89.916) (width 0.762) (layer B.Cu) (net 2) (status 400000))
 (segment (start 134.874 87.376) (end 134.874 88.2396) (width 0.762) (layer F.Cu) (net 2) (status 400000))
 (segment (start 138.379202 88.950798) (end 139.954 87.376) (width 0.762) (layer F.Cu) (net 2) (status 800000))
 (segment (start 135.585198 88.950798) (end 138.379202 88.950798) (width 0.762) (layer F.Cu) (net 2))
 (segment (start 134.874 88.2396) (end 135.585198 88.950798) (width 0.762) (layer F.Cu) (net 2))
 (segment (start 151.384 87.376) (end 151.384 88.2142) (width 0.762) (layer F.Cu) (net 2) (status 400000))
 (segment (start 155.0162 88.8238) (end 156.464 87.376) (width 0.762) (layer F.Cu) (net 2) (status 800000))
 (segment (start 151.9936 88.8238) (end 155.0162 88.8238) (width 0.762) (layer F.Cu) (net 2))
 (segment (start 151.384 88.2142) (end 151.9936 88.8238) (width 0.762) (layer F.Cu) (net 2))
 (segment (start 153.416 62.484) (end 153.416 66.326) (width 0.762) (layer F.Cu) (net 2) (status C00000))
 (segment (start 153.416 66.326) (end 152.686 67.056) (width 0.762) (layer F.Cu) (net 2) (status C00000))
 (segment (start 156.3878 85.4456) (end 156.3878 85.09) (width 0.25) (layer F.Cu) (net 7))
 (segment (start 155.6766 86.1568) (end 156.3878 85.4456) (width 0.25) (layer F.Cu) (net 7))
 (segment (start 148.844 86.1568) (end 155.6766 86.1568) (width 0.25) (layer F.Cu) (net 7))
 (segment (start 132.334 87.376) (end 132.4102 87.376) (width 0.25) (layer F.Cu) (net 7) (status C00000))
 (segment (start 148.844 84.7852) (end 148.844 86.1568) (width 0.25) (layer F.Cu) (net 7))
 (segment (start 148.844 86.1568) (end 148.844 87.376) (width 0.25) (layer F.Cu) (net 7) (status 800000))
 (segment (start 147.6502 83.5914) (end 148.844 84.7852) (width 0.25) (layer F.Cu) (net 7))
 (segment (start 140.6652 83.5914) (end 147.6502 83.5914) (width 0.25) (layer F.Cu) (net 7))
 (segment (start 140.0048 84.2518) (end 140.6652 83.5914) (width 0.25) (layer F.Cu) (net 7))
 (segment (start 140.0048 85.4202) (end 140.0048 84.2518) (width 0.25) (layer F.Cu) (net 7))
 (segment (start 139.3698 86.0552) (end 140.0048 85.4202) (width 0.25) (layer F.Cu) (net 7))
 (segment (start 133.731 86.0552) (end 139.3698 86.0552) (width 0.25) (layer F.Cu) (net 7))
 (segment (start 132.4102 87.376) (end 133.731 86.0552) (width 0.25) (layer F.Cu) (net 7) (status 400000))
 (segment (start 156.3878 85.09) (end 156.3878 82.9818) (width 0.25) (layer F.Cu) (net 7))
 (segment (start 149.098 72.39) (end 147.32 72.39) (width 0.25) (layer F.Cu) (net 7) (status 800000))
 (segment (start 149.606 72.898) (end 149.098 72.39) (width 0.25) (layer F.Cu) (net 7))
 (segment (start 149.606 79.248) (end 149.606 72.898) (width 0.25) (layer F.Cu) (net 7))
 (segment (start 151.638 81.28) (end 149.606 79.248) (width 0.25) (layer F.Cu) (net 7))
 (segment (start 154.686 81.28) (end 151.638 81.28) (width 0.25) (layer F.Cu) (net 7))
 (segment (start 156.3878 82.9818) (end 154.686 81.28) (width 0.25) (layer F.Cu) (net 7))
 (segment (start 147.32 72.39) (end 147.32 67.564) (width 0.25) (layer F.Cu) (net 7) (status C00000))
 (segment (start 147.32 67.564) (end 147.828 67.056) (width 0.25) (layer F.Cu) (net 7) (status C00000))
 (segment (start 150.114 83.0072) (end 150.114 84.836) (width 0.25) (layer B.Cu) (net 6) (status 800000))
 (segment (start 149.2504 82.1436) (end 150.114 83.0072) (width 0.25) (layer B.Cu) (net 6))
 (segment (start 134.0104 82.1436) (end 142.24 82.1436) (width 0.25) (layer B.Cu) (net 6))
 (segment (start 133.604 82.55) (end 134.0104 82.1436) (width 0.25) (layer B.Cu) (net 6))
 (segment (start 133.604 84.836) (end 133.604 82.55) (width 0.25) (layer B.Cu) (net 6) (status 400000))
 (segment (start 142.24 82.1436) (end 147.32 82.1436) (width 0.25) (layer B.Cu) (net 6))
 (segment (start 147.32 82.1436) (end 149.2504 82.1436) (width 0.25) (layer B.Cu) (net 6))
 (segment (start 137.544 66.802) (end 141.986 66.802) (width 0.25) (layer F.Cu) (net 6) (status C00000))
 (segment (start 141.986 66.802) (end 142.24 67.056) (width 0.25) (layer F.Cu) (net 6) (status C00000))
 (segment (start 142.24 67.056) (end 142.24 82.1436) (width 0.25) (layer B.Cu) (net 6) (status 400000))
 (segment (start 142.24 82.1436) (end 142.24 82.042) (width 0.25) (layer B.Cu) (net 6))
 (segment (start 142.24 82.042) (end 142.24 82.1436) (width 0.25) (layer B.Cu) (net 6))
 (segment (start 136.144 84.836) (end 136.144 83.185) (width 0.25) (layer B.Cu) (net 5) (status 400000))
 (segment (start 151.384 86.106) (end 152.654 84.836) (width 0.25) (layer B.Cu) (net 5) (status 800000))
 (segment (start 149.2758 86.106) (end 151.384 86.106) (width 0.25) (layer B.Cu) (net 5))
 (segment (start 148.717 85.5472) (end 149.2758 86.106) (width 0.25) (layer B.Cu) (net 5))
 (segment (start 148.717 83.7438) (end 148.717 85.5472) (width 0.25) (layer B.Cu) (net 5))
 (segment (start 147.6502 82.677) (end 148.717 83.7438) (width 0.25) (layer B.Cu) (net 5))
 (segment (start 136.652 82.677) (end 147.6502 82.677) (width 0.25) (layer B.Cu) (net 5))
 (segment (start 136.144 83.185) (end 136.652 82.677) (width 0.25) (layer B.Cu) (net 5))
 (segment (start 137.414 87.376) (end 137.414 88.3412) (width 0.25) (layer B.Cu) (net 4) (status 400000))
 (segment (start 153.924 88.3666) (end 153.924 87.376) (width 0.25) (layer B.Cu) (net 4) (status 800000))
 (segment (start 153.289 89.0016) (end 153.924 88.3666) (width 0.25) (layer B.Cu) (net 4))
 (segment (start 138.0744 89.0016) (end 153.289 89.0016) (width 0.25) (layer B.Cu) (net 4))
 (segment (start 137.414 88.3412) (end 138.0744 89.0016) (width 0.25) (layer B.Cu) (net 4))
 (segment (start 138.684 84.836) (end 138.684 83.7438) (width 0.25) (layer F.Cu) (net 3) (status 400000))
 (segment (start 155.194 83.4644) (end 155.194 84.836) (width 0.25) (layer F.Cu) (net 3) (status 800000))
 (segment (start 154.7622 83.0326) (end 155.194 83.4644) (width 0.25) (layer F.Cu) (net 3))
 (segment (start 139.3952 83.0326) (end 154.7622 83.0326) (width 0.25) (layer F.Cu) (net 3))
 (segment (start 138.684 83.7438) (end 139.3952 83.0326) (width 0.25) (layer F.Cu) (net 3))
 (segment (start 156.3 75) (end 156.3 67.442) (width 0.762) (layer F.Cu) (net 9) (status C00000))
 (segment (start 156.3 67.442) (end 156.686 67.056) (width 0.762) (layer F.Cu) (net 9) (status C00000))
 (segment (start 133.7 75) (end 133.7 76.0928) (width 0.762) (layer F.Cu) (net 10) (status C00000))
 (segment (start 138.1252 80.518) (end 140.3565 80.518) (width 0.762) (layer F.Cu) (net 10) (status 800000))
 (segment (start 133.7 76.0928) (end 138.1252 80.518) (width 0.762) (layer F.Cu) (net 10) (status 400000))
 (segment (start 134.744 66.802) (end 132.842 66.802) (width 0.25) (layer F.Cu) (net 11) (status 400000))
 (segment (start 145.288 74.93) (end 147.32 74.93) (width 0.25) (layer B.Cu) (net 11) (status 800000))
 (segment (start 144.78 74.422) (end 145.288 74.93) (width 0.25) (layer B.Cu) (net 11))
 (segment (start 144.78 67.056) (end 144.78 74.422) (width 0.25) (layer B.Cu) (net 11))
 (segment (start 143.002 65.278) (end 144.78 67.056) (width 0.25) (layer B.Cu) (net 11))
 (segment (start 134.366 65.278) (end 143.002 65.278) (width 0.25) (layer B.Cu) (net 11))
 (segment (start 132.842 66.802) (end 134.366 65.278) (width 0.25) (layer B.Cu) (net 11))
 (via (at 132.842 66.802) (size 0.8) (drill 0.4) (layers F.Cu B.Cu) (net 11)))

